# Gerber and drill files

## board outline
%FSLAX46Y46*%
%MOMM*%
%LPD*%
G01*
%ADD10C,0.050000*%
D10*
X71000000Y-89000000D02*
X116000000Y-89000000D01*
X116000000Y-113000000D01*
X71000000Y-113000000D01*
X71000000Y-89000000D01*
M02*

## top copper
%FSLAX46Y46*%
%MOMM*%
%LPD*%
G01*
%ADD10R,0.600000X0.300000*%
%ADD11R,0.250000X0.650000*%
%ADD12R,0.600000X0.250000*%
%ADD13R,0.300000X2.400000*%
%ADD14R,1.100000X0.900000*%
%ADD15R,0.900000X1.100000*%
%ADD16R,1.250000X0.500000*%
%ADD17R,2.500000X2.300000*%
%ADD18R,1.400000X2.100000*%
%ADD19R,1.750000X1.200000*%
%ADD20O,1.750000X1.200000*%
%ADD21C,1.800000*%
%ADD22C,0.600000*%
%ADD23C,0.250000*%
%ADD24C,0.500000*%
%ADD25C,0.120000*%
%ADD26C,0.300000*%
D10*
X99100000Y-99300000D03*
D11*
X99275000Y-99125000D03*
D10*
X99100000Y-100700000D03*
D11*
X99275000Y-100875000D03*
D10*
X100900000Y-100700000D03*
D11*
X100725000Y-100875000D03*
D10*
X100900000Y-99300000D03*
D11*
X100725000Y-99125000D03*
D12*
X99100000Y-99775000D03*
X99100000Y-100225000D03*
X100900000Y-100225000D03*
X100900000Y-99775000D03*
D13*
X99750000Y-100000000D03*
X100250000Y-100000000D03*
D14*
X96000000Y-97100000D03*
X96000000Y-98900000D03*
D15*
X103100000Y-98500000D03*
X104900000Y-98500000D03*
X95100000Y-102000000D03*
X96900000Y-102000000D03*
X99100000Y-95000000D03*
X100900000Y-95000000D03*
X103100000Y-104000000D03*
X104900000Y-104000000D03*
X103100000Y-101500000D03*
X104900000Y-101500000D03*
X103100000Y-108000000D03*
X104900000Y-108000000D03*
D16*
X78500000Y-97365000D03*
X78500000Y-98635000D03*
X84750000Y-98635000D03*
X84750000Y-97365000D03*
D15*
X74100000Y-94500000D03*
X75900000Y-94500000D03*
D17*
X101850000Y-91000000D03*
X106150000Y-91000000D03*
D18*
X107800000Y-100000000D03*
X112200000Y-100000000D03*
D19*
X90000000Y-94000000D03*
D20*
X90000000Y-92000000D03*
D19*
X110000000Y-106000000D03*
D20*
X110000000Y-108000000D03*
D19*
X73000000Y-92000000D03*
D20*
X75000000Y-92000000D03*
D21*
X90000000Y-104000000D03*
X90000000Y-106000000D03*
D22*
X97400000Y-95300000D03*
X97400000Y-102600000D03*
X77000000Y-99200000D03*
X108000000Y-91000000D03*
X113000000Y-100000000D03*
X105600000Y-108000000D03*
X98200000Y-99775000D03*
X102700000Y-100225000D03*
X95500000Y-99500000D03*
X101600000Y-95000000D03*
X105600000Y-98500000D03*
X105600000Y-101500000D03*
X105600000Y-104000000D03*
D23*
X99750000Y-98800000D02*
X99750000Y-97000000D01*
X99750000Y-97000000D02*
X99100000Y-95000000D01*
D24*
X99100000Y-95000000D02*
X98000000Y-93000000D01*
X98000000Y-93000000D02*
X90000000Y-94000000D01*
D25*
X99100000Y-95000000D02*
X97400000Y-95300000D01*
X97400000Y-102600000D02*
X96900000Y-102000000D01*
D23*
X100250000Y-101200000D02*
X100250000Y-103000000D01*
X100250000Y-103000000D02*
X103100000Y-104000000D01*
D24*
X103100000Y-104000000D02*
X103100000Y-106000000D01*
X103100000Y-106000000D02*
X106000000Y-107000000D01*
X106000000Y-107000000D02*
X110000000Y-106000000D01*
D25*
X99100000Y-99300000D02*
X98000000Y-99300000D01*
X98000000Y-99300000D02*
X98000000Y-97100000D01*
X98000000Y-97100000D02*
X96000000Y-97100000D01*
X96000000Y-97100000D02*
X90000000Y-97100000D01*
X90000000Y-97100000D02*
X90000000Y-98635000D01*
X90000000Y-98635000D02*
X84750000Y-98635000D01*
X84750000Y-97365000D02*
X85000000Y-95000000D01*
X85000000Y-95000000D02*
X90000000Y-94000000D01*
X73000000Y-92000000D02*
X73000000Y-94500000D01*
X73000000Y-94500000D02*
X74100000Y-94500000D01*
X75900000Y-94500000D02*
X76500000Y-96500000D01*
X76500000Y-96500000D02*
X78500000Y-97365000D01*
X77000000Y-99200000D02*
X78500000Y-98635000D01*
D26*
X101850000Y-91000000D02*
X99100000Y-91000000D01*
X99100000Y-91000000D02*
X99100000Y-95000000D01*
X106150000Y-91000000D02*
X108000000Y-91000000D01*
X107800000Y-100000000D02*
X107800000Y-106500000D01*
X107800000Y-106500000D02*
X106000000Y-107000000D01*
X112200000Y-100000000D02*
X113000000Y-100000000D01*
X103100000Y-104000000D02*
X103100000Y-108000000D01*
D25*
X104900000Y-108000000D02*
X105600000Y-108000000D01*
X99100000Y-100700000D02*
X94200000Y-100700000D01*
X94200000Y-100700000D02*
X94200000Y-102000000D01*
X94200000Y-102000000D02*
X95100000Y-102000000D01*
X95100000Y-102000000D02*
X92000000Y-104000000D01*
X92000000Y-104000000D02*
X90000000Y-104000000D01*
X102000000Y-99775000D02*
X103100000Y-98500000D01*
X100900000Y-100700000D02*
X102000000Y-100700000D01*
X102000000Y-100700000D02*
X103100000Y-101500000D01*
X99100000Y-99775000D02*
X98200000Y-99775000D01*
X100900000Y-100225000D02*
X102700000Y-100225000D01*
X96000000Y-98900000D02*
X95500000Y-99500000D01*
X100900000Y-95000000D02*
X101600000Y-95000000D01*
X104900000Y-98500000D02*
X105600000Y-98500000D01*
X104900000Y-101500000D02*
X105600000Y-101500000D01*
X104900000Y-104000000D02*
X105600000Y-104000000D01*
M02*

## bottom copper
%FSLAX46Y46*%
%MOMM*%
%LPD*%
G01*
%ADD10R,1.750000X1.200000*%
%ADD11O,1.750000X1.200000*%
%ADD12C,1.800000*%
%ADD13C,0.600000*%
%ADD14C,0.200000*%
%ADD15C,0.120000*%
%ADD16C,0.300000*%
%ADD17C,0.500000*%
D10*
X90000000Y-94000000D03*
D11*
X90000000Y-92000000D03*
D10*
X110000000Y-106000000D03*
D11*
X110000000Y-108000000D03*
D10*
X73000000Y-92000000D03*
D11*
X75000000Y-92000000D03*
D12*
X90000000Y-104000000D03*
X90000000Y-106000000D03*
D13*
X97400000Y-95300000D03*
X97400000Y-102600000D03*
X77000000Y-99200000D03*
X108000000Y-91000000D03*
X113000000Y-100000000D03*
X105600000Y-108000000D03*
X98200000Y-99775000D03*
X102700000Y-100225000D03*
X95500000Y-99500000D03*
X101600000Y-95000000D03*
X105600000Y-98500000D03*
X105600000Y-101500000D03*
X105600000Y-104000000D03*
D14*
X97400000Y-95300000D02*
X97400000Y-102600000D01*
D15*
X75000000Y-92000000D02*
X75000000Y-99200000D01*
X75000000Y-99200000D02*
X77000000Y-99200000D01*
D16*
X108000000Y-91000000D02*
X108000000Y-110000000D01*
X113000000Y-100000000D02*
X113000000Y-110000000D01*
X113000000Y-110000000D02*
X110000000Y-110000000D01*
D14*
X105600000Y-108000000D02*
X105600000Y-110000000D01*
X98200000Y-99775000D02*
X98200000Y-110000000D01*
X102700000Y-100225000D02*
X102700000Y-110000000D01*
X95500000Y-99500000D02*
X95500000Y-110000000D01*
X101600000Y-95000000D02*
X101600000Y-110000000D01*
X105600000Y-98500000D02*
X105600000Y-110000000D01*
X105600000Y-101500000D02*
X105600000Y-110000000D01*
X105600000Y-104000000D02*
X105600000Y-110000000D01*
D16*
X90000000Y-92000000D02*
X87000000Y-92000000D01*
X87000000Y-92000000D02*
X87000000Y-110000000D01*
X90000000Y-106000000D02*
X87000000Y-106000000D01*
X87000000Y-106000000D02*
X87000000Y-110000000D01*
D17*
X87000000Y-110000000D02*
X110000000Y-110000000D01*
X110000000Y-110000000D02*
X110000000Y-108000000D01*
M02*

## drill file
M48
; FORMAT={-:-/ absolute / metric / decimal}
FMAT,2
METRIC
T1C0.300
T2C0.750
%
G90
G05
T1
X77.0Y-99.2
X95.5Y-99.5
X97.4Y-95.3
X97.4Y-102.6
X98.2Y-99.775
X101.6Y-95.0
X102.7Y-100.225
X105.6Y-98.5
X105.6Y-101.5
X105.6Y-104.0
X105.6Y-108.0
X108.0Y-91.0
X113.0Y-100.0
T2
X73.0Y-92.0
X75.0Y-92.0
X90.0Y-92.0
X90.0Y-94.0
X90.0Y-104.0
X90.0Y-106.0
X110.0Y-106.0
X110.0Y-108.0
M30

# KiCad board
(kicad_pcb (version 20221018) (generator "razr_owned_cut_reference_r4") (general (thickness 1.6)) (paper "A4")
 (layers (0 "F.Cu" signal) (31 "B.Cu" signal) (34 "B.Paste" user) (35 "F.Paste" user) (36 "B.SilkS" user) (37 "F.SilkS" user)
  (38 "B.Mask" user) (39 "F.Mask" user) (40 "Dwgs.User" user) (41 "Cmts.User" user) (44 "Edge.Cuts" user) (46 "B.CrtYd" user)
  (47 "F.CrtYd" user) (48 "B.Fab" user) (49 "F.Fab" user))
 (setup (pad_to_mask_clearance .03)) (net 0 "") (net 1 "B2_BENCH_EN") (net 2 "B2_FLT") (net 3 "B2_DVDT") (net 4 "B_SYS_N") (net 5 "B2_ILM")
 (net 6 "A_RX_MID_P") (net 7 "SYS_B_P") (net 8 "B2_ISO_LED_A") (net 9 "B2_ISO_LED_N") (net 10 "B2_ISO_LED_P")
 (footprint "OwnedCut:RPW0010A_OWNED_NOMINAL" (layer "F.Cu") (at 100 100)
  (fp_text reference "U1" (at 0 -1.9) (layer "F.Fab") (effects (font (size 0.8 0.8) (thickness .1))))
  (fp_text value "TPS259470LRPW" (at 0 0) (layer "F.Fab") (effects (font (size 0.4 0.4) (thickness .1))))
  (pad "1" smd rect (at -0.9 -0.7) (size 0.6 0.3) (layers "F.Cu" "F.Paste" "F.Mask") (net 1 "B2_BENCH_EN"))
  (pad "1" smd rect (at -0.725 -0.875) (size 0.25 0.65) (layers "F.Cu" "F.Paste" "F.Mask") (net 1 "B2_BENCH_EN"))
  (pad "4" smd rect (at -0.9 0.7) (size 0.6 0.3) (layers "F.Cu" "F.Paste" "F.Mask") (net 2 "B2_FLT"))
  (pad "4" smd rect (at -0.725 0.875) (size 0.25 0.65) (layers "F.Cu" "F.Paste" "F.Mask") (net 2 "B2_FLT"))
  (pad "7" smd rect (at 0.9 0.7) (size 0.6 0.3) (layers "F.Cu" "F.Paste" "F.Mask") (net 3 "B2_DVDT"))
  (pad "7" smd rect (at 0.725 0.875) (size 0.25 0.65) (layers "F.Cu" "F.Paste" "F.Mask") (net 3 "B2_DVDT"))
  (pad "10" smd rect (at 0.9 -0.7) (size 0.6 0.3) (layers "F.Cu" "F.Paste" "F.Mask"))
  (pad "10" smd rect (at 0.725 -0.875) (size 0.25 0.65) (layers "F.Cu" "F.Paste" "F.Mask"))
  (pad "2" smd rect (at -0.9 -0.225) (size 0.6 0.25) (layers "F.Cu" "F.Paste" "F.Mask") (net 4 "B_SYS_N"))
  (pad "3" smd rect (at -0.9 0.225) (size 0.6 0.25) (layers "F.Cu" "F.Paste" "F.Mask"))
  (pad "8" smd rect (at 0.9 0.225) (size 0.6 0.25) (layers "F.Cu" "F.Paste" "F.Mask") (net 4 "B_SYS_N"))
  (pad "9" smd rect (at 0.9 -0.225) (size 0.6 0.25) (layers "F.Cu" "F.Paste" "F.Mask") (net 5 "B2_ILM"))
  (pad "5" smd rect (at -0.25 0) (size 0.3 2.4) (layers "F.Cu" "F.Paste" "F.Mask") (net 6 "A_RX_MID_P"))
  (pad "6" smd rect (at 0.25 0) (size 0.3 2.4) (layers "F.Cu" "F.Paste" "F.Mask") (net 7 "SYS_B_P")))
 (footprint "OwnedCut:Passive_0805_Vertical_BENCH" (layer "F.Cu") (at 96 98)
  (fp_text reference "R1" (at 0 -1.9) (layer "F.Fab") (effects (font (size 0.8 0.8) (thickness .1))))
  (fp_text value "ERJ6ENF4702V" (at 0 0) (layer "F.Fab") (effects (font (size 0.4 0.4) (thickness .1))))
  (pad "1" smd rect (at 0 -0.9) (size 1.1 0.9) (layers "F.Cu" "F.Paste" "F.Mask") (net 1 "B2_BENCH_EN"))
  (pad "2" smd rect (at 0 0.9) (size 1.1 0.9) (layers "F.Cu" "F.Paste" "F.Mask") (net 4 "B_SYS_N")))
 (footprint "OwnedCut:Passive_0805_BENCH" (layer "F.Cu") (at 104 98.5)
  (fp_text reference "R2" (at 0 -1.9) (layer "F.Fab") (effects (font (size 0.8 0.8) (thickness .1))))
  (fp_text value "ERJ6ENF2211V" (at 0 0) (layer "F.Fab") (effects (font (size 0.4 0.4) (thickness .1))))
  (pad "1" smd rect (at -0.9 0) (size 0.9 1.1) (layers "F.Cu" "F.Paste" "F.Mask") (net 5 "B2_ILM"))
  (pad "2" smd rect (at 0.9 0) (size 0.9 1.1) (layers "F.Cu" "F.Paste" "F.Mask") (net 4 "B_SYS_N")))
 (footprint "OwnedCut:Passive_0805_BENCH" (layer "F.Cu") (at 96 102)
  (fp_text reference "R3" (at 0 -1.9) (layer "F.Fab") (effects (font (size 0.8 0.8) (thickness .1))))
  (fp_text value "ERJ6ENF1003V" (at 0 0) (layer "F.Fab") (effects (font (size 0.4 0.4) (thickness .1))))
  (pad "1" smd rect (at -0.9 0) (size 0.9 1.1) (layers "F.Cu" "F.Paste" "F.Mask") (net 2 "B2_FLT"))
  (pad "2" smd rect (at 0.9 0) (size 0.9 1.1) (layers "F.Cu" "F.Paste" "F.Mask") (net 6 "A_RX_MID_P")))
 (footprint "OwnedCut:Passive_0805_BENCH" (layer "F.Cu") (at 100 95)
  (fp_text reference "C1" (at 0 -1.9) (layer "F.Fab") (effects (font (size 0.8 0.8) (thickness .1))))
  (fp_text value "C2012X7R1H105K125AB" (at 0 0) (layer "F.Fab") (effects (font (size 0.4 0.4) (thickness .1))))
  (pad "1" smd rect (at -0.9 0) (size 0.9 1.1) (layers "F.Cu" "F.Paste" "F.Mask") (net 6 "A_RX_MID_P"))
  (pad "2" smd rect (at 0.9 0) (size 0.9 1.1) (layers "F.Cu" "F.Paste" "F.Mask") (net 4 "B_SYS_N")))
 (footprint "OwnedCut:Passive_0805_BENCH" (layer "F.Cu") (at 104 104)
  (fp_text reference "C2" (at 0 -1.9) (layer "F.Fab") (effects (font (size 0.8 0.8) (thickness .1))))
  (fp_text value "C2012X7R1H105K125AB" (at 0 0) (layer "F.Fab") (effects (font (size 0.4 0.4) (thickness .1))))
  (pad "1" smd rect (at -0.9 0) (size 0.9 1.1) (layers "F.Cu" "F.Paste" "F.Mask") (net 7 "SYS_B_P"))
  (pad "2" smd rect (at 0.9 0) (size 0.9 1.1) (layers "F.Cu" "F.Paste" "F.Mask") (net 4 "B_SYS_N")))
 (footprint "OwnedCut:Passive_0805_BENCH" (layer "F.Cu") (at 104 101.5)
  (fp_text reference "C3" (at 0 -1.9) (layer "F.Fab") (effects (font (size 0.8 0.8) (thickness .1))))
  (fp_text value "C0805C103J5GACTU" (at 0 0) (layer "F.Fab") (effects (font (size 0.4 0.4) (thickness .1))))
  (pad "1" smd rect (at -0.9 0) (size 0.9 1.1) (layers "F.Cu" "F.Paste" "F.Mask") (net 3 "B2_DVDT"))
  (pad "2" smd rect (at 0.9 0) (size 0.9 1.1) (layers "F.Cu" "F.Paste" "F.Mask") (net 4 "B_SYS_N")))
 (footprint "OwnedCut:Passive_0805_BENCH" (layer "F.Cu") (at 104 108)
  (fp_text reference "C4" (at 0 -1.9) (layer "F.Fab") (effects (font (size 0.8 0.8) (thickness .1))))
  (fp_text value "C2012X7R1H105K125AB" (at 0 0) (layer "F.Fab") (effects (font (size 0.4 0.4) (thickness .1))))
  (pad "1" smd rect (at -0.9 0) (size 0.9 1.1) (layers "F.Cu" "F.Paste" "F.Mask") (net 7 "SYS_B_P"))
  (pad "2" smd rect (at 0.9 0) (size 0.9 1.1) (layers "F.Cu" "F.Paste" "F.Mask") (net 4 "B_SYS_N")))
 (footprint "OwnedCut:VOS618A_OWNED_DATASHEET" (layer "F.Cu") (at 81.625 98)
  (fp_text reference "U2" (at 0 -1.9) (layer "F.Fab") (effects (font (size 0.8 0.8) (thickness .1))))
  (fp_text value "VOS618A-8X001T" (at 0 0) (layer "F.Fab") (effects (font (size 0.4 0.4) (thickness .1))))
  (pad "1" smd rect (at -3.125 -0.635) (size 1.25 0.5) (layers "F.Cu" "F.Paste" "F.Mask") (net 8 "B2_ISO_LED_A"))
  (pad "2" smd rect (at -3.125 0.635) (size 1.25 0.5) (layers "F.Cu" "F.Paste" "F.Mask") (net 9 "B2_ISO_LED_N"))
  (pad "3" smd rect (at 3.125 0.635) (size 1.25 0.5) (layers "F.Cu" "F.Paste" "F.Mask") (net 1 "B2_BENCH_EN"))
  (pad "4" smd rect (at 3.125 -0.635) (size 1.25 0.5) (layers "F.Cu" "F.Paste" "F.Mask") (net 6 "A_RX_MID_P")))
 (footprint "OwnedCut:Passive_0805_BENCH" (layer "F.Cu") (at 75 94.5)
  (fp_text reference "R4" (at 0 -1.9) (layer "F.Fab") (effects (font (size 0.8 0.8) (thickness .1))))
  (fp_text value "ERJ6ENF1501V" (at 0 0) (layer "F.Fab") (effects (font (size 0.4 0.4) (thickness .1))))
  (pad "1" smd rect (at -0.9 0) (size 0.9 1.1) (layers "F.Cu" "F.Paste" "F.Mask") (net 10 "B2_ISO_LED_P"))
  (pad "2" smd rect (at 0.9 0) (size 0.9 1.1) (layers "F.Cu" "F.Paste" "F.Mask") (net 8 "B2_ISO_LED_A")))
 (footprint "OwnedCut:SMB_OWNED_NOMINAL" (layer "F.Cu") (at 104 91)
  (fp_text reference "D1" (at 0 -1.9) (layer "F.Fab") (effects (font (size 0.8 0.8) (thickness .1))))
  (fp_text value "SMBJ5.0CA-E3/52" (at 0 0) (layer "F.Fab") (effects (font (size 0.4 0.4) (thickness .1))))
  (pad "1" smd rect (at -2.15 0) (size 2.5 2.3) (layers "F.Cu" "F.Paste" "F.Mask") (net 6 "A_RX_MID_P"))
  (pad "2" smd rect (at 2.15 0) (size 2.5 2.3) (layers "F.Cu" "F.Paste" "F.Mask") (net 4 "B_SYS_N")))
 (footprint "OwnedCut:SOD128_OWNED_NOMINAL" (layer "F.Cu") (at 110 100)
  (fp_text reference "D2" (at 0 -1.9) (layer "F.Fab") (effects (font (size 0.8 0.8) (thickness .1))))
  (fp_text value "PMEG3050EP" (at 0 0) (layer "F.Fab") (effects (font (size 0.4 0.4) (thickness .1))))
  (pad "1" smd rect (at -2.2 0) (size 1.4 2.1) (layers "F.Cu" "F.Paste" "F.Mask") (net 7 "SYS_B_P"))
  (pad "2" smd rect (at 2.2 0) (size 1.4 2.1) (layers "F.Cu" "F.Paste" "F.Mask") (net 4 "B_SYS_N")))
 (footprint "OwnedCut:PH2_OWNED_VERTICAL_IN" (layer "F.Cu") (at 90 94)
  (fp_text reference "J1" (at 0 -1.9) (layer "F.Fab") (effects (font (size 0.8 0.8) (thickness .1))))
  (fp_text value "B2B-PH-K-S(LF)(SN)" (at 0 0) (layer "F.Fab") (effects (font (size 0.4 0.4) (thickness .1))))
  (pad "1" thru_hole rect (at 0 0) (size 1.75 1.2) (drill .75) (layers "*.Cu" "*.Mask") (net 6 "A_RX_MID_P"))
  (pad "2" thru_hole oval (at 0 -2) (size 1.75 1.2) (drill .75) (layers "*.Cu" "*.Mask") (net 4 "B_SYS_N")))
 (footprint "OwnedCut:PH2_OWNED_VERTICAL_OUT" (layer "F.Cu") (at 110 106)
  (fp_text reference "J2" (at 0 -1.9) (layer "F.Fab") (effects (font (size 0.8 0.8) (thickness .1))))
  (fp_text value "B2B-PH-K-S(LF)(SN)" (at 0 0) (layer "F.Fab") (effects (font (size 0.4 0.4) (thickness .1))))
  (pad "1" thru_hole rect (at 0 0) (size 1.75 1.2) (drill .75) (layers "*.Cu" "*.Mask") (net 7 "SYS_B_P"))
  (pad "2" thru_hole oval (at 0 2) (size 1.75 1.2) (drill .75) (layers "*.Cu" "*.Mask") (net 4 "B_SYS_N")))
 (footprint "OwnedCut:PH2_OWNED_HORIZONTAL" (layer "F.Cu") (at 73 92)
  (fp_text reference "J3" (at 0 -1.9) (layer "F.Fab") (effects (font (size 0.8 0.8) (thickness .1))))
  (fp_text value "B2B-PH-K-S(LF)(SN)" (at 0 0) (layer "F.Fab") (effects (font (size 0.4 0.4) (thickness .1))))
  (pad "1" thru_hole rect (at 0 0) (size 1.75 1.2) (drill .75) (layers "*.Cu" "*.Mask") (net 10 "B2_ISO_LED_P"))
  (pad "2" thru_hole oval (at 2 0) (size 1.75 1.2) (drill .75) (layers "*.Cu" "*.Mask") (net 9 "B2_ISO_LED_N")))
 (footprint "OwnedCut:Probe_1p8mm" (layer "F.Cu") (at 90 104)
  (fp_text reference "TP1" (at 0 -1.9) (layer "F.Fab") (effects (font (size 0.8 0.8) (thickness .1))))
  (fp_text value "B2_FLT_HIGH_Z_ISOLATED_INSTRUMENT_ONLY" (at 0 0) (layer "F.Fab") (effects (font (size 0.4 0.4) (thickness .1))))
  (pad "1" thru_hole circle (at 0 0) (size 1.8 1.8) (drill .75) (layers "*.Cu" "*.Mask") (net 2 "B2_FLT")))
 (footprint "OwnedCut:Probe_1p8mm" (layer "F.Cu") (at 90 106)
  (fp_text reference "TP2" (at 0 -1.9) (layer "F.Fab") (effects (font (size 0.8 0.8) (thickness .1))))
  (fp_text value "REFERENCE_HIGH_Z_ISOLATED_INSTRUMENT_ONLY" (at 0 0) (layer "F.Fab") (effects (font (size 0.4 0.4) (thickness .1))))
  (pad "1" thru_hole circle (at 0 0) (size 1.8 1.8) (drill .75) (layers "*.Cu" "*.Mask") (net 4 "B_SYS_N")))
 (segment (start 99.75 98.8) (end 99.75 97) (width 0.25) (layer "F.Cu") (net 6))
 (segment (start 99.75 97) (end 99.1 95) (width 0.25) (layer "F.Cu") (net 6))
 (segment (start 99.1 95) (end 98 93) (width 0.5) (layer "F.Cu") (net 6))
 (segment (start 98 93) (end 90 94) (width 0.5) (layer "F.Cu") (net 6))
 (segment (start 99.1 95) (end 97.4 95.3) (width 0.12) (layer "F.Cu") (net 6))
 (via (at 97.4 95.3) (size .6) (drill .3) (layers "F.Cu" "B.Cu") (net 6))
 (segment (start 97.4 95.3) (end 97.4 102.6) (width 0.2) (layer "B.Cu") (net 6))
 (via (at 97.4 102.6) (size .6) (drill .3) (layers "F.Cu" "B.Cu") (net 6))
 (segment (start 97.4 102.6) (end 96.9 102) (width 0.12) (layer "F.Cu") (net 6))
 (segment (start 100.25 101.2) (end 100.25 103) (width 0.25) (layer "F.Cu") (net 7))
 (segment (start 100.25 103) (end 103.1 104) (width 0.25) (layer "F.Cu") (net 7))
 (segment (start 103.1 104) (end 103.1 106) (width 0.5) (layer "F.Cu") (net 7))
 (segment (start 103.1 106) (end 106 107) (width 0.5) (layer "F.Cu") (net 7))
 (segment (start 106 107) (end 110 106) (width 0.5) (layer "F.Cu") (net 7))
 (segment (start 99.1 99.3) (end 98 99.3) (width 0.12) (layer "F.Cu") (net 1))
 (segment (start 98 99.3) (end 98 97.1) (width 0.12) (layer "F.Cu") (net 1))
 (segment (start 98 97.1) (end 96 97.1) (width 0.12) (layer "F.Cu") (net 1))
 (segment (start 96 97.1) (end 90 97.1) (width 0.12) (layer "F.Cu") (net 1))
 (segment (start 90 97.1) (end 90 98.635) (width 0.12) (layer "F.Cu") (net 1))
 (segment (start 90 98.635) (end 84.75 98.635) (width 0.12) (layer "F.Cu") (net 1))
 (segment (start 84.75 97.365) (end 85 95) (width 0.12) (layer "F.Cu") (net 6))
 (segment (start 85 95) (end 90 94) (width 0.12) (layer "F.Cu") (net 6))
 (segment (start 73 92) (end 73 94.5) (width 0.12) (layer "F.Cu") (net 10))
 (segment (start 73 94.5) (end 74.1 94.5) (width 0.12) (layer "F.Cu") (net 10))
 (segment (start 75.9 94.5) (end 76.5 96.5) (width 0.12) (layer "F.Cu") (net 8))
 (segment (start 76.5 96.5) (end 78.5 97.365) (width 0.12) (layer "F.Cu") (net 8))
 (segment (start 75 92) (end 75 99.2) (width 0.12) (layer "B.Cu") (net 9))
 (segment (start 75 99.2) (end 77 99.2) (width 0.12) (layer "B.Cu") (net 9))
 (via (at 77 99.2) (size .6) (drill .3) (layers "F.Cu" "B.Cu") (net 9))
 (segment (start 77 99.2) (end 78.5 98.635) (width 0.12) (layer "F.Cu") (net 9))
 (segment (start 101.85 91) (end 99.1 91) (width 0.3) (layer "F.Cu") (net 6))
 (segment (start 99.1 91) (end 99.1 95) (width 0.3) (layer "F.Cu") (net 6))
 (segment (start 106.15 91) (end 108 91) (width 0.3) (layer "F.Cu") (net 4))
 (via (at 108 91) (size .6) (drill .3) (layers "F.Cu" "B.Cu") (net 4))
 (segment (start 108 91) (end 108 110) (width 0.3) (layer "B.Cu") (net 4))
 (segment (start 107.8 100) (end 107.8 106.5) (width 0.3) (layer "F.Cu") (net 7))
 (segment (start 107.8 106.5) (end 106 107) (width 0.3) (layer "F.Cu") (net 7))
 (segment (start 112.2 100) (end 113 100) (width 0.3) (layer "F.Cu") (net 4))
 (via (at 113 100) (size .6) (drill .3) (layers "F.Cu" "B.Cu") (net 4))
 (segment (start 113 100) (end 113 110) (width 0.3) (layer "B.Cu") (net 4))
 (segment (start 113 110) (end 110 110) (width 0.3) (layer "B.Cu") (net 4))
 (segment (start 103.1 104) (end 103.1 108) (width 0.3) (layer "F.Cu") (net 7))
 (segment (start 104.9 108) (end 105.6 108) (width 0.12) (layer "F.Cu") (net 4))
 (via (at 105.6 108) (size .6) (drill .3) (layers "F.Cu" "B.Cu") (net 4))
 (segment (start 105.6 108) (end 105.6 110) (width 0.2) (layer "B.Cu") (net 4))
 (segment (start 99.1 100.7) (end 94.2 100.7) (width 0.12) (layer "F.Cu") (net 2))
 (segment (start 94.2 100.7) (end 94.2 102) (width 0.12) (layer "F.Cu") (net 2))
 (segment (start 94.2 102) (end 95.1 102) (width 0.12) (layer "F.Cu") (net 2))
 (segment (start 95.1 102) (end 92 104) (width 0.12) (layer "F.Cu") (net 2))
 (segment (start 92 104) (end 90 104) (width 0.12) (layer "F.Cu") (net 2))
 (segment (start 102 99.775) (end 103.1 98.5) (width 0.12) (layer "F.Cu") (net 5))
 (segment (start 100.9 100.7) (end 102 100.7) (width 0.12) (layer "F.Cu") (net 3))
 (segment (start 102 100.7) (end 103.1 101.5) (width 0.12) (layer "F.Cu") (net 3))
 (segment (start 99.1 99.775) (end 98.2 99.775) (width 0.12) (layer "F.Cu") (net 4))
 (via (at 98.2 99.775) (size .6) (drill .3) (layers "F.Cu" "B.Cu") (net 4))
 (segment (start 98.2 99.775) (end 98.2 110) (width 0.2) (layer "B.Cu") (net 4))
 (segment (start 100.9 100.225) (end 102.7 100.225) (width 0.12) (layer "F.Cu") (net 4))
 (via (at 102.7 100.225) (size .6) (drill .3) (layers "F.Cu" "B.Cu") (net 4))
 (segment (start 102.7 100.225) (end 102.7 110) (width 0.2) (layer "B.Cu") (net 4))
 (segment (start 96 98.9) (end 95.5 99.5) (width 0.12) (layer "F.Cu") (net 4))
 (via (at 95.5 99.5) (size .6) (drill .3) (layers "F.Cu" "B.Cu") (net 4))
 (segment (start 95.5 99.5) (end 95.5 110) (width 0.2) (layer "B.Cu") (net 4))
 (segment (start 100.9 95) (end 101.6 95) (width 0.12) (layer "F.Cu") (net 4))
 (via (at 101.6 95) (size .6) (drill .3) (layers "F.Cu" "B.Cu") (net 4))
 (segment (start 101.6 95) (end 101.6 110) (width 0.2) (layer "B.Cu") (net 4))
 (segment (start 104.9 98.5) (end 105.6 98.5) (width 0.12) (layer "F.Cu") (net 4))
 (via (at 105.6 98.5) (size .6) (drill .3) (layers "F.Cu" "B.Cu") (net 4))
 (segment (start 105.6 98.5) (end 105.6 110) (width 0.2) (layer "B.Cu") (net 4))
 (segment (start 104.9 101.5) (end 105.6 101.5) (width 0.12) (layer "F.Cu") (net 4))
 (via (at 105.6 101.5) (size .6) (drill .3) (layers "F.Cu" "B.Cu") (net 4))
 (segment (start 105.6 101.5) (end 105.6 110) (width 0.2) (layer "B.Cu") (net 4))
 (segment (start 104.9 104) (end 105.6 104) (width 0.12) (layer "F.Cu") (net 4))
 (via (at 105.6 104) (size .6) (drill .3) (layers "F.Cu" "B.Cu") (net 4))
 (segment (start 105.6 104) (end 105.6 110) (width 0.2) (layer "B.Cu") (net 4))
 (segment (start 90 92) (end 87 92) (width 0.3) (layer "B.Cu") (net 4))
 (segment (start 87 92) (end 87 110) (width 0.3) (layer "B.Cu") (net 4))
 (segment (start 90 106) (end 87 106) (width 0.3) (layer "B.Cu") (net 4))
 (segment (start 87 106) (end 87 110) (width 0.3) (layer "B.Cu") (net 4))
 (segment (start 87 110) (end 110 110) (width 0.5) (layer "B.Cu") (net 4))
 (segment (start 110 110) (end 110 108) (width 0.5) (layer "B.Cu") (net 4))
 (gr_rect (start 71 89) (end 116 113) (stroke (width .05) (type default)) (fill none) (layer "Edge.Cuts")))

